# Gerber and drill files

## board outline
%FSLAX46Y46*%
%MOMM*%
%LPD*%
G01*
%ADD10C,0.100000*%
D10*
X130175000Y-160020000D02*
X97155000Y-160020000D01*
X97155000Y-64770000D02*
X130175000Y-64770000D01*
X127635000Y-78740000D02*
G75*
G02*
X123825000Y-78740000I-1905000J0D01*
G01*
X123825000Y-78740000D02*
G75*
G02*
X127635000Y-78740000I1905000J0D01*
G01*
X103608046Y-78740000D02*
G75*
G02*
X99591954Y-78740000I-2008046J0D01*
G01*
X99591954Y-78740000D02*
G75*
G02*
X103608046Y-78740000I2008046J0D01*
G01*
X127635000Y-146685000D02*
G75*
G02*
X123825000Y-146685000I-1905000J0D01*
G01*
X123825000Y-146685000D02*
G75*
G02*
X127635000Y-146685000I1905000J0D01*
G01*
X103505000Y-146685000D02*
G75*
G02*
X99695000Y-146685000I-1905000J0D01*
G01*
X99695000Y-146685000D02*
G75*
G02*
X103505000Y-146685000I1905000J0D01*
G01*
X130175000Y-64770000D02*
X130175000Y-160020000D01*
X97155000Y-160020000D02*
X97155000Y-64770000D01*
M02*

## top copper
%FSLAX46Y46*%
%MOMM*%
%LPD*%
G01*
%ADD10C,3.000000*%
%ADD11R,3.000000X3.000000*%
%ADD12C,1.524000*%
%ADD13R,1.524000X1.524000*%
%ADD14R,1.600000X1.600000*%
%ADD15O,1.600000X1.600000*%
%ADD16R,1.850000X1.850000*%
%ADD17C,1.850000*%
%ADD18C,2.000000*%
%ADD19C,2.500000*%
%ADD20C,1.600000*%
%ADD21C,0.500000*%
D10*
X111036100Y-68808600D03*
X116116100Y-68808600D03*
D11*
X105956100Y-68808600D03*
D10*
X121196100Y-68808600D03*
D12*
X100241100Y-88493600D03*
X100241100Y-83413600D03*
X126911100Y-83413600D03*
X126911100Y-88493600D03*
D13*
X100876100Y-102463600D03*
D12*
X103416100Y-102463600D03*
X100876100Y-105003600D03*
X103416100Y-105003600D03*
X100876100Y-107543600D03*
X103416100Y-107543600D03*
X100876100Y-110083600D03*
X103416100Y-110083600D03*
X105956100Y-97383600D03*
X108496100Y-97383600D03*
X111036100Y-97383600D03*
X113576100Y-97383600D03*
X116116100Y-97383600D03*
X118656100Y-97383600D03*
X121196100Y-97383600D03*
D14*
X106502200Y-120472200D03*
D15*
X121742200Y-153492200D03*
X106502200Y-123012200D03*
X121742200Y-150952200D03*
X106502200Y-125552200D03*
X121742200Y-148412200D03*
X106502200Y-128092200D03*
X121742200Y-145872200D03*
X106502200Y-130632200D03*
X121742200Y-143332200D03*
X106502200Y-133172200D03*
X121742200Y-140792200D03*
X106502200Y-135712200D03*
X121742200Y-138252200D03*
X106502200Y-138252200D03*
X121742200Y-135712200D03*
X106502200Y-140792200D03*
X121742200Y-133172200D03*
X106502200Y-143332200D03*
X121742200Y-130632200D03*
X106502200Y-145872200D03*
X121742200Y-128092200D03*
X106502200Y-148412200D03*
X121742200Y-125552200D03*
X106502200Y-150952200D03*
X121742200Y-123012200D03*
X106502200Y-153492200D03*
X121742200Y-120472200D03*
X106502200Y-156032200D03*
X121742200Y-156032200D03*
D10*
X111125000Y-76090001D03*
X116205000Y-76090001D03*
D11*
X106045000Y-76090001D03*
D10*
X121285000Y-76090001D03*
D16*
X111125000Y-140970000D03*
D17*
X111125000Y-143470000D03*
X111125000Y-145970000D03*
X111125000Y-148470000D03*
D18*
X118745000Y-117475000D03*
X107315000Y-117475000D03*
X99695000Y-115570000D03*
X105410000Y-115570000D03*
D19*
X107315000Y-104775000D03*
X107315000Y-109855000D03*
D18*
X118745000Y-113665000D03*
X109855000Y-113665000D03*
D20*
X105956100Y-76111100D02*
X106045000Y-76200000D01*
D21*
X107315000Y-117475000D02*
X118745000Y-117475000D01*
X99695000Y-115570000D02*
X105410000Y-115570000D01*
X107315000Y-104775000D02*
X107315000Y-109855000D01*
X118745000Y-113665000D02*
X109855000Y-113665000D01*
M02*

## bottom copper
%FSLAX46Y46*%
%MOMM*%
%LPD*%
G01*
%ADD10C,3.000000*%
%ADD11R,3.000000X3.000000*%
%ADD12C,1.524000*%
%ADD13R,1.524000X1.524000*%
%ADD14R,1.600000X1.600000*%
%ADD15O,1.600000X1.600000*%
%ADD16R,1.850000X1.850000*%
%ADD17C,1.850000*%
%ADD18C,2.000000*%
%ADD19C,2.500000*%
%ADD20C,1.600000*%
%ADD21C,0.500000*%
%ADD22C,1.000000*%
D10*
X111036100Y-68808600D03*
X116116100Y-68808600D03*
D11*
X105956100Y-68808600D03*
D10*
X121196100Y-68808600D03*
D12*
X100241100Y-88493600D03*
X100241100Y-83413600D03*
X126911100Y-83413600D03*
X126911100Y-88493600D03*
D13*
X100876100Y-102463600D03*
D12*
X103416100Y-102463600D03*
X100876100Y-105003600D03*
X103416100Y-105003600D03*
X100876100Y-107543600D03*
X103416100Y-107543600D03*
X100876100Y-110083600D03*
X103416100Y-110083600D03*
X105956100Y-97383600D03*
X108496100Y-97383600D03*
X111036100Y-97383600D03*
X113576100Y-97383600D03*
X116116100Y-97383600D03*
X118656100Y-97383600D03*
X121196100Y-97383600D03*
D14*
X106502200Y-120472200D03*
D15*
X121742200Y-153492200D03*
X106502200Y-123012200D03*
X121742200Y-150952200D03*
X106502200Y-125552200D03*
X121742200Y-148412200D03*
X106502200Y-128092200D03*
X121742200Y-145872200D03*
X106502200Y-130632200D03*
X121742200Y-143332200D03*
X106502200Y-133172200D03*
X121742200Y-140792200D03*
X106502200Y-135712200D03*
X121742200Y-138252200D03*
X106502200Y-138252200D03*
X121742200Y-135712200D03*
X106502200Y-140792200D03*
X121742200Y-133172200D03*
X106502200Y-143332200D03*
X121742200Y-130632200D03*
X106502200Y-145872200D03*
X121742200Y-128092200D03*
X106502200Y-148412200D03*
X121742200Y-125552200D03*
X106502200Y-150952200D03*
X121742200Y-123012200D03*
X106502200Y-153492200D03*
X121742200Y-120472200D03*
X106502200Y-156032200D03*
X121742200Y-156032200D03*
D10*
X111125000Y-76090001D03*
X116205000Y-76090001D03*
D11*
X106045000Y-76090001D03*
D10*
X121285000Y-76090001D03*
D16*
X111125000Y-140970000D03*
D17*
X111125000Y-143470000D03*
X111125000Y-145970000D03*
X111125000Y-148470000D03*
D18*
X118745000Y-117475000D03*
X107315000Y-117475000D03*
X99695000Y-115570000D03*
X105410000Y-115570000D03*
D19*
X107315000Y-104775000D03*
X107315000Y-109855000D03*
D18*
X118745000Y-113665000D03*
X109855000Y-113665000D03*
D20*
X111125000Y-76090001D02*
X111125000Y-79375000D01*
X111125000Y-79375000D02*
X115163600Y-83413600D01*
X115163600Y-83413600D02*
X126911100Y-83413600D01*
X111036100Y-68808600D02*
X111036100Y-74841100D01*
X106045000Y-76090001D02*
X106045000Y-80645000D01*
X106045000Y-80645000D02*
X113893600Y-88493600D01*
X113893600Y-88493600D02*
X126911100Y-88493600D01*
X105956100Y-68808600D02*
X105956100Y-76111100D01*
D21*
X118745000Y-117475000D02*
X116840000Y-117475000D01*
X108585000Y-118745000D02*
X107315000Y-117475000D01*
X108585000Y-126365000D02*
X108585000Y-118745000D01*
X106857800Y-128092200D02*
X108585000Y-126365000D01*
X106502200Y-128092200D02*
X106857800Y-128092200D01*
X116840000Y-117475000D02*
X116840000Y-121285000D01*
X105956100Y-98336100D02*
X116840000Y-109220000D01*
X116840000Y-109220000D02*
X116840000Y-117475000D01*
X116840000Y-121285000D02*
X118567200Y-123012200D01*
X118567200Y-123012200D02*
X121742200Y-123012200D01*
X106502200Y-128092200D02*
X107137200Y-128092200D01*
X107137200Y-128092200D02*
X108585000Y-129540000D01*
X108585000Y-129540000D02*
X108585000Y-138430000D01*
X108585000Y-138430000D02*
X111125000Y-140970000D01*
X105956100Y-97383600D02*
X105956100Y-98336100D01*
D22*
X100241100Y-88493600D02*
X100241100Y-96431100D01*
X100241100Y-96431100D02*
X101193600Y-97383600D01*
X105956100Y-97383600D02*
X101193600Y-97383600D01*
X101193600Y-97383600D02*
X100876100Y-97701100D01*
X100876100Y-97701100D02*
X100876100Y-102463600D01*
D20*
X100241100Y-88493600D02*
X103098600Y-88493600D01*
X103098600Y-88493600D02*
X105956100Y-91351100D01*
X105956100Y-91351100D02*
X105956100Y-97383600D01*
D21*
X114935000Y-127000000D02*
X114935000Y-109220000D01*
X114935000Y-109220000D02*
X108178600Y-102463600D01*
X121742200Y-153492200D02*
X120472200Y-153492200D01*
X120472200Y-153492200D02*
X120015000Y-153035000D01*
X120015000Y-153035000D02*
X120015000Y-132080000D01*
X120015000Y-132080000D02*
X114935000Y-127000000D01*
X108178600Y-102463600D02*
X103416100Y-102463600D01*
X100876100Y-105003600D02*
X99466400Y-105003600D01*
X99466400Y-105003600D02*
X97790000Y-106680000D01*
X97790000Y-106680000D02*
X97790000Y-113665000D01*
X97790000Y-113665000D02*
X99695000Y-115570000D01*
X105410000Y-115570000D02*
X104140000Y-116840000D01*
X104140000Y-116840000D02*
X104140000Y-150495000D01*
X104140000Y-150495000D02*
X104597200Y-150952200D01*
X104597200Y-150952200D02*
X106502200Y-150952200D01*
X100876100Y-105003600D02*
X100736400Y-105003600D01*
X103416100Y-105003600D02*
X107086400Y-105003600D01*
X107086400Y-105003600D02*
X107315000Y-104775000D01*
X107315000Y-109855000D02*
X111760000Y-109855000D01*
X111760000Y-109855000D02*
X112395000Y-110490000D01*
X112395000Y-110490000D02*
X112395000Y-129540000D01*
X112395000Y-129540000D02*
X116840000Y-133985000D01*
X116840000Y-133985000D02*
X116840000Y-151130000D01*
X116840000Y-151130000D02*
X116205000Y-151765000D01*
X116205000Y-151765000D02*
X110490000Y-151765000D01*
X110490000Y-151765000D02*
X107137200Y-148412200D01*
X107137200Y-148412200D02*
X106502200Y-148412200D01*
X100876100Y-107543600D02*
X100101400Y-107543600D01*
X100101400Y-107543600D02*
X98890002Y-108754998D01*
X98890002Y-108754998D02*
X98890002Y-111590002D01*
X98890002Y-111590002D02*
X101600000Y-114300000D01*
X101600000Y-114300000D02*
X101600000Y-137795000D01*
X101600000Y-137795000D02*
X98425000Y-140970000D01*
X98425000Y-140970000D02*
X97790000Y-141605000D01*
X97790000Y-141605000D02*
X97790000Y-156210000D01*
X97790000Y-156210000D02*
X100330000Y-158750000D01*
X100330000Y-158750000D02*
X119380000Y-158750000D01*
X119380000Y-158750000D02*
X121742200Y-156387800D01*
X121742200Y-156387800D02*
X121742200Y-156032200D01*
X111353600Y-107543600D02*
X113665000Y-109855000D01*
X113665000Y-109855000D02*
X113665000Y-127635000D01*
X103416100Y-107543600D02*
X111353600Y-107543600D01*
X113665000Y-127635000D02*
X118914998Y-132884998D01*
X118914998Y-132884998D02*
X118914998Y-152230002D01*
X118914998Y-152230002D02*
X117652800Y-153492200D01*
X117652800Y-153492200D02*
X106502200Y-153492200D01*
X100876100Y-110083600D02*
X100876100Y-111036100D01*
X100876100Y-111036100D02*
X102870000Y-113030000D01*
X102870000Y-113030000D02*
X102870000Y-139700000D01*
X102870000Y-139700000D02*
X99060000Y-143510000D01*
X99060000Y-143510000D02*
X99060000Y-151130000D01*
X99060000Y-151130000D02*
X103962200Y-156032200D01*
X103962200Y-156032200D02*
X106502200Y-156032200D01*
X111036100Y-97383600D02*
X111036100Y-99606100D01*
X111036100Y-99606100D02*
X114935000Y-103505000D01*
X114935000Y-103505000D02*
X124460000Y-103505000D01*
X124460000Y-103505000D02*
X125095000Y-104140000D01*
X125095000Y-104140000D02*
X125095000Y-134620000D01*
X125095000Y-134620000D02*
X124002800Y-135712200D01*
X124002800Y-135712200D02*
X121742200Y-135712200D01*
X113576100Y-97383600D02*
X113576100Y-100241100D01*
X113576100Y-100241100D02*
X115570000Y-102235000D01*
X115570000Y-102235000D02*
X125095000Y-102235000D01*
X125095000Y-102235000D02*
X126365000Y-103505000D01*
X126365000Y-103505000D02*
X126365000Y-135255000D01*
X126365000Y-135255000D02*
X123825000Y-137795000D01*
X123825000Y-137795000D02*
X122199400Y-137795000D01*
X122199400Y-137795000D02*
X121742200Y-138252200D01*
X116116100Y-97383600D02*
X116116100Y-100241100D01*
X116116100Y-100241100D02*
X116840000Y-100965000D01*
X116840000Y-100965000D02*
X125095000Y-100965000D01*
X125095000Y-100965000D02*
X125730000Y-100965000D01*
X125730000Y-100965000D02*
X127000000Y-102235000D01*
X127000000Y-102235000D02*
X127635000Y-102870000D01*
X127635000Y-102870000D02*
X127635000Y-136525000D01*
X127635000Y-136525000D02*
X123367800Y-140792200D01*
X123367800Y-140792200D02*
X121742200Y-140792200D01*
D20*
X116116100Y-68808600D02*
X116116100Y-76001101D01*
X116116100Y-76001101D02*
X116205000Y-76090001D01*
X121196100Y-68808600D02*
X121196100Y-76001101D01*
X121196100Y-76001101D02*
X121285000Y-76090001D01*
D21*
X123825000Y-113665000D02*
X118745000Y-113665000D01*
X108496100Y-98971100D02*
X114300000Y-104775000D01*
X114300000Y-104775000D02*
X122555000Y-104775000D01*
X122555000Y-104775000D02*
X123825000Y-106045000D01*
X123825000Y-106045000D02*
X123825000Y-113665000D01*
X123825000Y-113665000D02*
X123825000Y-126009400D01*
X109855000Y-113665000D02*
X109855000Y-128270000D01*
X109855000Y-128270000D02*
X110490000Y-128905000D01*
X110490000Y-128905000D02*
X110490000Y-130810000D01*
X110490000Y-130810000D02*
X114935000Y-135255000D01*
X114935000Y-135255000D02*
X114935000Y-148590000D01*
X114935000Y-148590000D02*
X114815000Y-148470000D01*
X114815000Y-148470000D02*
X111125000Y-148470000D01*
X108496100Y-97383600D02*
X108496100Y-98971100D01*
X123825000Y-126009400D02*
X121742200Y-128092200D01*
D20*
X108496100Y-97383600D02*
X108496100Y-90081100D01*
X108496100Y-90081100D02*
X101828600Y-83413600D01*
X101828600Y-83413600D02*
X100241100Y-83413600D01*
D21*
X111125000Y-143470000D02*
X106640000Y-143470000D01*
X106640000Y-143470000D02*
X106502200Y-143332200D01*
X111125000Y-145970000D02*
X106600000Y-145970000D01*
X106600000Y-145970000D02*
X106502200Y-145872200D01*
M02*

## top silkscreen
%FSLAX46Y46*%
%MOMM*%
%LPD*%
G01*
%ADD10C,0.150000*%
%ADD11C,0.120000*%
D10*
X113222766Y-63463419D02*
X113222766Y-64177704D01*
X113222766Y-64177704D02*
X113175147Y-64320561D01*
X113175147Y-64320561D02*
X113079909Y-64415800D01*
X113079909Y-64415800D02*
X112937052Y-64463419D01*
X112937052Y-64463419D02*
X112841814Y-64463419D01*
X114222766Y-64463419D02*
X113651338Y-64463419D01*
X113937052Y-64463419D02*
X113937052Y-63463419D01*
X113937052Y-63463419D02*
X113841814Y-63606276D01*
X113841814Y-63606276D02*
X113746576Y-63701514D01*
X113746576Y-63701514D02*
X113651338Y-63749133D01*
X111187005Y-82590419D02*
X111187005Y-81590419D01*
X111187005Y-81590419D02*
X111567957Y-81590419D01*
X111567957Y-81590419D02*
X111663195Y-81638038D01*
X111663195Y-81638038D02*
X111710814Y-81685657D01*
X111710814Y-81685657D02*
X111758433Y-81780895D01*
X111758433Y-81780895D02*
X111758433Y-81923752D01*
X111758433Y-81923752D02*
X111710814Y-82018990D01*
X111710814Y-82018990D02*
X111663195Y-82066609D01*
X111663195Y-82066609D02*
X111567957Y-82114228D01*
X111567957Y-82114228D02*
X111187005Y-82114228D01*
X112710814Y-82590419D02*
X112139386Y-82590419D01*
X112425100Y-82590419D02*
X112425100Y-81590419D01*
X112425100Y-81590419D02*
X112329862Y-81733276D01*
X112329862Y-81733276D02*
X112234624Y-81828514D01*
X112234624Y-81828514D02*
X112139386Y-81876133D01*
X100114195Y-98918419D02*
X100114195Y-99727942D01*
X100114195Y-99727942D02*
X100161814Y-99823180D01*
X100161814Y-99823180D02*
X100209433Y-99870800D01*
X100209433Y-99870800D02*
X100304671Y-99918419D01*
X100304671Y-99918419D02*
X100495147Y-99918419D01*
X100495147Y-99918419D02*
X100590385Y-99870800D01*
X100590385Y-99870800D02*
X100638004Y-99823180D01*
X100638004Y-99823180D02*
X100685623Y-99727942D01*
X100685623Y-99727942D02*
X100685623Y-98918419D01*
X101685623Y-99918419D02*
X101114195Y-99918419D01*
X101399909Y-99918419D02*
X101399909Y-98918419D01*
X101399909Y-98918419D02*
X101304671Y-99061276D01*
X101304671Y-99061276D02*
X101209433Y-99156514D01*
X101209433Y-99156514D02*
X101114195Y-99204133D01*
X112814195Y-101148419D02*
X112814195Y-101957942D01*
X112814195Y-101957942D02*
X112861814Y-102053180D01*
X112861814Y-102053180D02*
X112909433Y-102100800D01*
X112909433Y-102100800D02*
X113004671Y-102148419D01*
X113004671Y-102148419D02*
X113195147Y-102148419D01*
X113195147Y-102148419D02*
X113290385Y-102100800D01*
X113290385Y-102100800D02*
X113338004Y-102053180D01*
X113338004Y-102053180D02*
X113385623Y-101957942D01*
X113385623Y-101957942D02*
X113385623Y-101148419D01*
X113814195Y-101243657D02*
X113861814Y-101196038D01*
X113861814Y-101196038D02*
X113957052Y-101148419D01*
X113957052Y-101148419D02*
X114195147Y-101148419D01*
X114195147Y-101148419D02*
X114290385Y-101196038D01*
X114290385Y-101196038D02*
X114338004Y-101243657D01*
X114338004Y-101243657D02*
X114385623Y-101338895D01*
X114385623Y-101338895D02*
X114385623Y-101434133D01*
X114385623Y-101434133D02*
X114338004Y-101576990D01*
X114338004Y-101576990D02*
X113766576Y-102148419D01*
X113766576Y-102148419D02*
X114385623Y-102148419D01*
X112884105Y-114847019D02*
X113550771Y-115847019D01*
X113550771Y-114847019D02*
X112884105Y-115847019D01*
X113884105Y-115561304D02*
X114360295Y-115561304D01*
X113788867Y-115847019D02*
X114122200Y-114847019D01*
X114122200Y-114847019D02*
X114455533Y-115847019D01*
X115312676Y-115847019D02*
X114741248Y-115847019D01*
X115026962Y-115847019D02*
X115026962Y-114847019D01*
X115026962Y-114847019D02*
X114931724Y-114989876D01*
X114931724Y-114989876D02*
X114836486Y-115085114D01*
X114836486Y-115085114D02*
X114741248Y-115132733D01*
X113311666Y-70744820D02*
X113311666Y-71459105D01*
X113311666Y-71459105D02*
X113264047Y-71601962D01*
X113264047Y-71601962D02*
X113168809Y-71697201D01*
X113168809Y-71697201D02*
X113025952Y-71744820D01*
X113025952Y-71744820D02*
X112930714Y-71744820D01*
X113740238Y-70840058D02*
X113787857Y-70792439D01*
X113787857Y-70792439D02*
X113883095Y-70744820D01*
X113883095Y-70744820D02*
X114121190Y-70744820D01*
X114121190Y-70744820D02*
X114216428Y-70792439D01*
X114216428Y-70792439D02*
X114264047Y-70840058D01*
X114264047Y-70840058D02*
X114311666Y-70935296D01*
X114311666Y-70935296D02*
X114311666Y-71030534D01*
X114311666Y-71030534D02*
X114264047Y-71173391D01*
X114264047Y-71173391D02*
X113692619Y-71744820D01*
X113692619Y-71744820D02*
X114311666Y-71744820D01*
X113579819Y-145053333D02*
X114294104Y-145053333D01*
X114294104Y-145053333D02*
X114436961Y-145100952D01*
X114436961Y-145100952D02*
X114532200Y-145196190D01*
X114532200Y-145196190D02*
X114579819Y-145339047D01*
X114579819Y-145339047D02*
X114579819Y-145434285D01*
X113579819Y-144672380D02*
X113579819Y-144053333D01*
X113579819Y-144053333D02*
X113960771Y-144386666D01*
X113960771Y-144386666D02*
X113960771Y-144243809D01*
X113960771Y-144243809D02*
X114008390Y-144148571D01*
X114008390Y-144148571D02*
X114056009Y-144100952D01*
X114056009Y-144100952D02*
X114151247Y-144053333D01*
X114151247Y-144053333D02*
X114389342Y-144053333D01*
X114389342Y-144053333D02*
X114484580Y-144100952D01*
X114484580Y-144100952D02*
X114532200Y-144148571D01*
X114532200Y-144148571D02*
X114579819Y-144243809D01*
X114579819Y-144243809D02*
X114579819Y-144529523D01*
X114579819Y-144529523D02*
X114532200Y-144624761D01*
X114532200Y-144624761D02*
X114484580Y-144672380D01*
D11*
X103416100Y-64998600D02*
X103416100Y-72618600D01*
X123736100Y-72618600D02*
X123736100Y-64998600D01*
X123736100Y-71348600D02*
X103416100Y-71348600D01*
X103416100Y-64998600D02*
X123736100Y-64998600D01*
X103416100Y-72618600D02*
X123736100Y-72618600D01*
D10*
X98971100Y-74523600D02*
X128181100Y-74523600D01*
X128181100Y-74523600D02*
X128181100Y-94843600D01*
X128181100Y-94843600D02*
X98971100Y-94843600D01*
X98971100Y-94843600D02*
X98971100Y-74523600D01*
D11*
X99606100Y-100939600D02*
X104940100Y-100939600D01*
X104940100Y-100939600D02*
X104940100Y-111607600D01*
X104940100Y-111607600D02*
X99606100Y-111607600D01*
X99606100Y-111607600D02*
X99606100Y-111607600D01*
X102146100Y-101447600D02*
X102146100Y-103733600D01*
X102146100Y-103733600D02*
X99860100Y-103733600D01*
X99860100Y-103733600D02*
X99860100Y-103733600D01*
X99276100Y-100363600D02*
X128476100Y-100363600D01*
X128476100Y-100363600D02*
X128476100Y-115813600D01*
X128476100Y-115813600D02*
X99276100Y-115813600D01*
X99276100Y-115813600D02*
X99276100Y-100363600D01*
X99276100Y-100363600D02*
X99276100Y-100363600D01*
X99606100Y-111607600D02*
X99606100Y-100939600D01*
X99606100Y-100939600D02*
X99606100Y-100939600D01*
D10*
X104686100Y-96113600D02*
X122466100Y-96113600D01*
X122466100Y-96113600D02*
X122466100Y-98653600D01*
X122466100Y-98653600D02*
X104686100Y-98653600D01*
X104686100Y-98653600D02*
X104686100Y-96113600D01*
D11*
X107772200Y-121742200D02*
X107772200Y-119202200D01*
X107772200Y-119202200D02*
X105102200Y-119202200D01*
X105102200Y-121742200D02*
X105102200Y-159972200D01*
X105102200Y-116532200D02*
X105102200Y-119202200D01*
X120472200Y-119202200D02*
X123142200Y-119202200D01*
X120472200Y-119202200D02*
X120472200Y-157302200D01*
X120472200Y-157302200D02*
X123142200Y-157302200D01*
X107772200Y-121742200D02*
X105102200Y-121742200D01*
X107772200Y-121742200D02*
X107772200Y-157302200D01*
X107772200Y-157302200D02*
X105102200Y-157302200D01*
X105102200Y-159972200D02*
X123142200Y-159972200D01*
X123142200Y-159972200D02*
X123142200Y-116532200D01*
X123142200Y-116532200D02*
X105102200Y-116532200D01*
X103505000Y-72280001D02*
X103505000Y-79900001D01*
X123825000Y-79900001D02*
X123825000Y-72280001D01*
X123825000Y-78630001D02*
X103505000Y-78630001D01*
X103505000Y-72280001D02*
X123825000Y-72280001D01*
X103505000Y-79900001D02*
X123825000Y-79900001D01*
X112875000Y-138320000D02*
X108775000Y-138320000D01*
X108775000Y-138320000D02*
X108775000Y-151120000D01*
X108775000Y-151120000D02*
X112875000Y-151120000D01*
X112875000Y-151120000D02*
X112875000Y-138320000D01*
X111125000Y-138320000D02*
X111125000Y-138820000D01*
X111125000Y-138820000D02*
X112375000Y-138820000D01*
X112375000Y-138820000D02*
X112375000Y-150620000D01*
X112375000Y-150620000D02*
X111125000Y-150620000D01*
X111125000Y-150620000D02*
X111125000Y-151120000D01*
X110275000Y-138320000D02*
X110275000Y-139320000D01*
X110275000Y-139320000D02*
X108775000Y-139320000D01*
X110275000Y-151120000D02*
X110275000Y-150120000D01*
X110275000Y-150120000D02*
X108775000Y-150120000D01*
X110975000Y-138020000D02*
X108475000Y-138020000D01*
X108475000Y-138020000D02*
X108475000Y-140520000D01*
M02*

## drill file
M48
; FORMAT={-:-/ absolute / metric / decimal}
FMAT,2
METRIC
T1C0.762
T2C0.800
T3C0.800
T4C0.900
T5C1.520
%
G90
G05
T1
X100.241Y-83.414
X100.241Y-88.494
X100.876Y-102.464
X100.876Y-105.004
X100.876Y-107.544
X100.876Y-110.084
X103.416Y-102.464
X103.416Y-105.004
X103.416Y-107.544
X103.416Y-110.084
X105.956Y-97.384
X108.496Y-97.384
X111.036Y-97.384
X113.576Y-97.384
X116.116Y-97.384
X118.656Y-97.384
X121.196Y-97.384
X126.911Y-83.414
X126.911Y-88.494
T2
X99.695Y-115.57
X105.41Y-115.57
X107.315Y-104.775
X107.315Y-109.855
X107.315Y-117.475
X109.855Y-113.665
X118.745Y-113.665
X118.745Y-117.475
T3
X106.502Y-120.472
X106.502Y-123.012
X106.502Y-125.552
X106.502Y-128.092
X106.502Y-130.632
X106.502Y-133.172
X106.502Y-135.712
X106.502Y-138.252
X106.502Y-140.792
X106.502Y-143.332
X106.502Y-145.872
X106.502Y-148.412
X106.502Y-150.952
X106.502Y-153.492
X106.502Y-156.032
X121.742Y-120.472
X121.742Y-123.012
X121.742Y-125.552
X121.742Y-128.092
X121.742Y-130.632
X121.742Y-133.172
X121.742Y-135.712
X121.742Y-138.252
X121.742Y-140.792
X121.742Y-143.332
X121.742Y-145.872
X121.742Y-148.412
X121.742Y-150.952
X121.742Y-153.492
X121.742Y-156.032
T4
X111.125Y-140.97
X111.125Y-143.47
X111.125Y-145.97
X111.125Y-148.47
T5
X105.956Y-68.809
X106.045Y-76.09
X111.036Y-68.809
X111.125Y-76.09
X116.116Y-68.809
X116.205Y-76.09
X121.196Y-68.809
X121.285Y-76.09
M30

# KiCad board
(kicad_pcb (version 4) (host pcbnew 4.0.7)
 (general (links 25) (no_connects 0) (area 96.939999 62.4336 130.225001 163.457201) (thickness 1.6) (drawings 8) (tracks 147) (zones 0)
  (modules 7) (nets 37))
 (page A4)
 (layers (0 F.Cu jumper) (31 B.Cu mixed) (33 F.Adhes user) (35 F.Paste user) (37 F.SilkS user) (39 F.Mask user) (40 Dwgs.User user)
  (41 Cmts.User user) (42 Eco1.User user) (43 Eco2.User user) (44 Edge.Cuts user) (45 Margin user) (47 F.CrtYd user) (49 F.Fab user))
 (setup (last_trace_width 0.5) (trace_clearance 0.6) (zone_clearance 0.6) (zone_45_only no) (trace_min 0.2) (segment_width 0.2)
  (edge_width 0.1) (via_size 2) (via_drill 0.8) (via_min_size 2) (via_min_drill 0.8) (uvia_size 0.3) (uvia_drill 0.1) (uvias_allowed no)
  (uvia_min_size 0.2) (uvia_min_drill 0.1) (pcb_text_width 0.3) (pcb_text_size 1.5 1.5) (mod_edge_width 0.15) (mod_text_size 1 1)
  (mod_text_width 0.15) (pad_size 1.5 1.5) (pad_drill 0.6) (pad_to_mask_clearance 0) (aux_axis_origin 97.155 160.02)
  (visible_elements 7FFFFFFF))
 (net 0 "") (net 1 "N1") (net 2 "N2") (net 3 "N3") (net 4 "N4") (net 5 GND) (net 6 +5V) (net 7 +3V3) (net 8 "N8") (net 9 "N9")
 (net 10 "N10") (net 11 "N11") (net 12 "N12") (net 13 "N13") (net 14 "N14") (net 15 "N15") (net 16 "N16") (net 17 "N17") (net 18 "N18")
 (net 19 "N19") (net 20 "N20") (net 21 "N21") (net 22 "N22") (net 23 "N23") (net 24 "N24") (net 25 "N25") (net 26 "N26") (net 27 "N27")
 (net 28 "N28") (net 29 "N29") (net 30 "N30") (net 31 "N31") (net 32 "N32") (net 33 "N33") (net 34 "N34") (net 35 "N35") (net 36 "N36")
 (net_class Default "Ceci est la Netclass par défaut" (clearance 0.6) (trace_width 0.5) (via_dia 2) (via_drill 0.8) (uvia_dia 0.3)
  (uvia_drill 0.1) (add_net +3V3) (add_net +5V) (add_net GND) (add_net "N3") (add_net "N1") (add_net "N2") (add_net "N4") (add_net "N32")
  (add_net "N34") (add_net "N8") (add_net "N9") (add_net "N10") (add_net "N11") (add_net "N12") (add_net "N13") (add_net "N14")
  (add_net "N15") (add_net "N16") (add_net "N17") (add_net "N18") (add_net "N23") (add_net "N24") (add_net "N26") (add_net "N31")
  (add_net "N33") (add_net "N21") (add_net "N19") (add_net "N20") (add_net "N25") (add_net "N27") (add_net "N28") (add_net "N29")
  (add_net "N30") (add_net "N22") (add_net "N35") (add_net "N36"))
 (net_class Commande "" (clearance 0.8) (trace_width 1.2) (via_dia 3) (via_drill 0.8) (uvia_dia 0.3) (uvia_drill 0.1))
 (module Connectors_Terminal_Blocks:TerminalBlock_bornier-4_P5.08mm (layer F.Cu) (at 105.9561 68.8086)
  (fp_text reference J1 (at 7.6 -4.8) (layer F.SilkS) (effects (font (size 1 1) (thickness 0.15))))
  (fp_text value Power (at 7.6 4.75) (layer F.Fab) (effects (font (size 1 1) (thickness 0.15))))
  (fp_line (start -2.54 -3.81) (end -2.54 3.81) (layer F.SilkS) (width 0.12))
  (fp_line (start 17.78 3.81) (end 17.78 -3.81) (layer F.SilkS) (width 0.12))
  (fp_line (start 17.78 2.54) (end -2.54 2.54) (layer F.SilkS) (width 0.12))
  (fp_line (start -2.54 -3.81) (end 17.78 -3.81) (layer F.SilkS) (width 0.12))
  (fp_line (start -2.54 3.81) (end 17.78 3.81) (layer F.SilkS) (width 0.12))
  (pad 2 thru_hole circle (at 5.08 0) (size 3 3) (drill 1.52) (layers *.Cu *.Mask) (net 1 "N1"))
  (pad 3 thru_hole circle (at 10.16 0) (size 3 3) (drill 1.52) (layers *.Cu *.Mask) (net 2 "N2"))
  (pad 1 thru_hole rect (at 0 0) (size 3 3) (drill 1.52) (layers *.Cu *.Mask) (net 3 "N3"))
  (pad 4 thru_hole circle (at 15.24 0) (size 3 3) (drill 1.52) (layers *.Cu *.Mask) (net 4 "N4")))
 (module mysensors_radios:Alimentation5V (layer F.Cu) (at 112.9411 84.6836)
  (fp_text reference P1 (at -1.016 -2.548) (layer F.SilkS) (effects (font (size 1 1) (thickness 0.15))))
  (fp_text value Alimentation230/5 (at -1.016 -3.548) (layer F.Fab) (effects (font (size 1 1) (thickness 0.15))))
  (fp_line (start -13.97 -10.16) (end 15.24 -10.16) (layer F.SilkS) (width 0.15))
  (fp_line (start 15.24 -10.16) (end 15.24 10.16) (layer F.SilkS) (width 0.15))
  (fp_line (start 15.24 10.16) (end -13.97 10.16) (layer F.SilkS) (width 0.15))
  (fp_line (start -13.97 10.16) (end -13.97 -10.16) (layer F.SilkS) (width 0.15))
  (pad 4 thru_hole circle (at -12.7 3.81) (size 1.524 1.524) (drill 0.762) (layers *.Cu *.Mask) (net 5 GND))
  (pad 3 thru_hole circle (at -12.7 -1.27) (size 1.524 1.524) (drill 0.762) (layers *.Cu *.Mask) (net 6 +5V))
  (pad 1 thru_hole circle (at 13.97 -1.27) (size 1.524 1.524) (drill 0.762) (layers *.Cu *.Mask) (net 1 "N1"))
  (pad 2 thru_hole circle (at 13.97 3.81) (size 1.524 1.524) (drill 0.762) (layers *.Cu *.Mask) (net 3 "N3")))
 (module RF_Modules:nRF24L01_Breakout (layer F.Cu) (at 100.8761 102.4636)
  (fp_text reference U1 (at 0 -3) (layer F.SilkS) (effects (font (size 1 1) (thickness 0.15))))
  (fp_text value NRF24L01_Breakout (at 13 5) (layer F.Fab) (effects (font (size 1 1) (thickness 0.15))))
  (fp_line (start -1.27 -1.524) (end 4.064 -1.524) (layer F.SilkS) (width 0.12))
  (fp_line (start 4.064 -1.524) (end 4.064 9.144) (layer F.SilkS) (width 0.12))
  (fp_line (start 4.064 9.144) (end -1.27 9.144) (layer F.SilkS) (width 0.12))
  (fp_line (start -1.27 9.144) (end -1.27 9.144) (layer F.SilkS) (width 0.12))
  (fp_line (start 1.27 -1.016) (end 1.27 1.27) (layer F.SilkS) (width 0.12))
  (fp_line (start 1.27 1.27) (end -1.016 1.27) (layer F.SilkS) (width 0.12))
  (fp_line (start -1.016 1.27) (end -1.016 1.27) (layer F.SilkS) (width 0.12))
  (fp_line (start -1.6 -2.1) (end 27.6 -2.1) (layer F.SilkS) (width 0.12))
  (fp_line (start 27.6 -2.1) (end 27.6 13.35) (layer F.SilkS) (width 0.12))
  (fp_line (start 27.6 13.35) (end -1.6 13.35) (layer F.SilkS) (width 0.12))
  (fp_line (start -1.6 13.35) (end -1.6 -2.1) (layer F.SilkS) (width 0.12))
  (fp_line (start -1.6 -2.1) (end -1.6 -2.1) (layer F.SilkS) (width 0.12))
  (fp_line (start -1.27 9.144) (end -1.27 -1.524) (layer F.SilkS) (width 0.12))
  (fp_line (start -1.27 -1.524) (end -1.27 -1.524) (layer F.SilkS) (width 0.12))
  (pad 1 thru_hole rect (at 0 0) (size 1.524 1.524) (drill 0.762) (layers *.Cu *.Mask) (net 5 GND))
  (pad 2 thru_hole circle (at 2.54 0) (size 1.524 1.524) (drill 0.762) (layers *.Cu *.Mask) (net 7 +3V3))
  (pad 3 thru_hole circle (at 0 2.54) (size 1.524 1.524) (drill 0.762) (layers *.Cu *.Mask) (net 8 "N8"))
  (pad 4 thru_hole circle (at 2.54 2.54) (size 1.524 1.524) (drill 0.762) (layers *.Cu *.Mask) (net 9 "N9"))
  (pad 5 thru_hole circle (at 0 5.08) (size 1.524 1.524) (drill 0.762) (layers *.Cu *.Mask) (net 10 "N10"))
  (pad 6 thru_hole circle (at 2.54 5.08) (size 1.524 1.524) (drill 0.762) (layers *.Cu *.Mask) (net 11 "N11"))
  (pad 7 thru_hole circle (at 0 7.62) (size 1.524 1.524) (drill 0.762) (layers *.Cu *.Mask) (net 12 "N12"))
  (pad 8 thru_hole circle (at 2.54 7.62) (size 1.524 1.524) (drill 0.762) (layers *.Cu *.Mask) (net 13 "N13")))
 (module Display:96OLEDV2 (layer F.Cu) (at 105.9561 97.3836)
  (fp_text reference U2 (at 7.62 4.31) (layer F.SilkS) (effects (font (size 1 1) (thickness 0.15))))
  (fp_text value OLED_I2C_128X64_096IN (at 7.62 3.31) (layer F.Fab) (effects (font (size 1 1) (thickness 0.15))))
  (fp_line (start -1.27 -1.27) (end 16.51 -1.27) (layer F.SilkS) (width 0.15))
  (fp_line (start 16.51 -1.27) (end 16.51 1.27) (layer F.SilkS) (width 0.15))
  (fp_line (start 16.51 1.27) (end -1.27 1.27) (layer F.SilkS) (width 0.15))
  (fp_line (start -1.27 1.27) (end -1.27 -1.27) (layer F.SilkS) (width 0.15))
  (pad 1 thru_hole circle (at 0 0) (size 1.524 1.524) (drill 0.762) (layers *.Cu *.Mask) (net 5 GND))
  (pad 2 thru_hole circle (at 2.54 0) (size 1.524 1.524) (drill 0.762) (layers *.Cu *.Mask) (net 6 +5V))
  (pad 3 thru_hole circle (at 5.08 0) (size 1.524 1.524) (drill 0.762) (layers *.Cu *.Mask) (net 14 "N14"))
  (pad 4 thru_hole circle (at 7.62 0) (size 1.524 1.524) (drill 0.762) (layers *.Cu *.Mask) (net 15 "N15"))
  (pad 5 thru_hole circle (at 10.16 0) (size 1.524 1.524) (drill 0.762) (layers *.Cu *.Mask) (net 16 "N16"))
  (pad 6 thru_hole circle (at 12.7 0) (size 1.524 1.524) (drill 0.762) (layers *.Cu *.Mask) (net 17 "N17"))
  (pad 7 thru_hole circle (at 15.24 0) (size 1.524 1.524) (drill 0.762) (layers *.Cu *.Mask) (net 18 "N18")))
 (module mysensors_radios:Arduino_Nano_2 (layer F.Cu) (at 106.5022 120.4722)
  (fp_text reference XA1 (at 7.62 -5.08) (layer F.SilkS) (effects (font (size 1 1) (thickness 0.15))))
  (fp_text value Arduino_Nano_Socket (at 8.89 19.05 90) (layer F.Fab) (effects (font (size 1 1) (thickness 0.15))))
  (fp_line (start 1.27 1.27) (end 1.27 -1.27) (layer F.SilkS) (width 0.12))
  (fp_line (start 1.27 -1.27) (end -1.4 -1.27) (layer F.SilkS) (width 0.12))
  (fp_line (start -1.4 1.27) (end -1.4 39.5) (layer F.SilkS) (width 0.12))
  (fp_line (start -1.4 -3.94) (end -1.4 -1.27) (layer F.SilkS) (width 0.12))
  (fp_line (start 13.97 -1.27) (end 16.64 -1.27) (layer F.SilkS) (width 0.12))
  (fp_line (start 13.97 -1.27) (end 13.97 36.83) (layer F.SilkS) (width 0.12))
  (fp_line (start 13.97 36.83) (end 16.64 36.83) (layer F.SilkS) (width 0.12))
  (fp_line (start 1.27 1.27) (end -1.4 1.27) (layer F.SilkS) (width 0.12))
  (fp_line (start 1.27 1.27) (end 1.27 36.83) (layer F.SilkS) (width 0.12))
  (fp_line (start 1.27 36.83) (end -1.4 36.83) (layer F.SilkS) (width 0.12))
  (fp_line (start -1.4 39.5) (end 16.64 39.5) (layer F.SilkS) (width 0.12))
  (fp_line (start 16.64 39.5) (end 16.64 -3.94) (layer F.SilkS) (width 0.12))
  (fp_line (start 16.64 -3.94) (end -1.4 -3.94) (layer F.SilkS) (width 0.12))
  (pad D0 thru_hole rect (at 0 0) (size 1.6 1.6) (drill 0.8) (layers *.Cu *.Mask) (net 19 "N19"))
  (pad 3V3 thru_hole oval (at 15.24 33.02) (size 1.6 1.6) (drill 0.8) (layers *.Cu *.Mask) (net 7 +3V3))
  (pad D1 thru_hole oval (at 0 2.54) (size 1.6 1.6) (drill 0.8) (layers *.Cu *.Mask) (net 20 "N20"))
  (pad AREF thru_hole oval (at 15.24 30.48) (size 1.6 1.6) (drill 0.8) (layers *.Cu *.Mask) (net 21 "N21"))
  (pad RST1 thru_hole oval (at 0 5.08) (size 1.6 1.6) (drill 0.8) (layers *.Cu *.Mask) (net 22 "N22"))
  (pad A0 thru_hole oval (at 15.24 27.94) (size 1.6 1.6) (drill 0.8) (layers *.Cu *.Mask) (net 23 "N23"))
  (pad GND1 thru_hole oval (at 0 7.62) (size 1.6 1.6) (drill 0.8) (layers *.Cu *.Mask) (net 5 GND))
  (pad A1 thru_hole oval (at 15.24 25.4) (size 1.6 1.6) (drill 0.8) (layers *.Cu *.Mask) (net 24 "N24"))
  (pad D2 thru_hole oval (at 0 10.16) (size 1.6 1.6) (drill 0.8) (layers *.Cu *.Mask) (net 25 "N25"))
  (pad A2 thru_hole oval (at 15.24 22.86) (size 1.6 1.6) (drill 0.8) (layers *.Cu *.Mask) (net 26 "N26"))
  (pad D3 thru_hole oval (at 0 12.7) (size 1.6 1.6) (drill 0.8) (layers *.Cu *.Mask) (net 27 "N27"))
  (pad A3 thru_hole oval (at 15.24 20.32) (size 1.6 1.6) (drill 0.8) (layers *.Cu *.Mask) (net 16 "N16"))
  (pad D4 thru_hole oval (at 0 15.24) (size 1.6 1.6) (drill 0.8) (layers *.Cu *.Mask) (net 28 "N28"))
  (pad A4 thru_hole oval (at 15.24 17.78) (size 1.6 1.6) (drill 0.8) (layers *.Cu *.Mask) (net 15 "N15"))
  (pad D5 thru_hole oval (at 0 17.78) (size 1.6 1.6) (drill 0.8) (layers *.Cu *.Mask) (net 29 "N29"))
  (pad A5 thru_hole oval (at 15.24 15.24) (size 1.6 1.6) (drill 0.8) (layers *.Cu *.Mask) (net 14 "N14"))
  (pad D6 thru_hole oval (at 0 20.32) (size 1.6 1.6) (drill 0.8) (layers *.Cu *.Mask) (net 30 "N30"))
  (pad A6 thru_hole oval (at 15.24 12.7) (size 1.6 1.6) (drill 0.8) (layers *.Cu *.Mask) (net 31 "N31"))
  (pad D7 thru_hole oval (at 0 22.86) (size 1.6 1.6) (drill 0.8) (layers *.Cu *.Mask) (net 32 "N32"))
  (pad A7 thru_hole oval (at 15.24 10.16) (size 1.6 1.6) (drill 0.8) (layers *.Cu *.Mask) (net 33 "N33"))
  (pad D8 thru_hole oval (at 0 25.4) (size 1.6 1.6) (drill 0.8) (layers *.Cu *.Mask) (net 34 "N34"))
  (pad 5V thru_hole oval (at 15.24 7.62) (size 1.6 1.6) (drill 0.8) (layers *.Cu *.Mask) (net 6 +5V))
  (pad D9 thru_hole oval (at 0 27.94) (size 1.6 1.6) (drill 0.8) (layers *.Cu *.Mask) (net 9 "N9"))
  (pad RST2 thru_hole oval (at 15.24 5.08) (size 1.6 1.6) (drill 0.8) (layers *.Cu *.Mask) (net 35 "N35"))
  (pad D10 thru_hole oval (at 0 30.48) (size 1.6 1.6) (drill 0.8) (layers *.Cu *.Mask) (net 8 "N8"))
  (pad GND2 thru_hole oval (at 15.24 2.54) (size 1.6 1.6) (drill 0.8) (layers *.Cu *.Mask) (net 5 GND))
  (pad D11 thru_hole oval (at 0 33.02) (size 1.6 1.6) (drill 0.8) (layers *.Cu *.Mask) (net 11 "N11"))
  (pad VIN thru_hole oval (at 15.24 0) (size 1.6 1.6) (drill 0.8) (layers *.Cu *.Mask) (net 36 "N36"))
  (pad D12 thru_hole oval (at 0 35.56) (size 1.6 1.6) (drill 0.8) (layers *.Cu *.Mask) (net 12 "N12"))
  (pad D13 thru_hole oval (at 15.24 35.56) (size 1.6 1.6) (drill 0.8) (layers *.Cu *.Mask) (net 10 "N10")))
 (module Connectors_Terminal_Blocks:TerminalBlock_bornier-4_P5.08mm (layer F.Cu) (at 106.045 76.090001)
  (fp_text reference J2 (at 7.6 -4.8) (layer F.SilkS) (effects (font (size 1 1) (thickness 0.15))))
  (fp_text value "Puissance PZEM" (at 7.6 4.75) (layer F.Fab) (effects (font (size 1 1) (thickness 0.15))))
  (fp_line (start -2.54 -3.81) (end -2.54 3.81) (layer F.SilkS) (width 0.12))
  (fp_line (start 17.78 3.81) (end 17.78 -3.81) (layer F.SilkS) (width 0.12))
  (fp_line (start 17.78 2.54) (end -2.54 2.54) (layer F.SilkS) (width 0.12))
  (fp_line (start -2.54 -3.81) (end 17.78 -3.81) (layer F.SilkS) (width 0.12))
  (fp_line (start -2.54 3.81) (end 17.78 3.81) (layer F.SilkS) (width 0.12))
  (pad 2 thru_hole circle (at 5.08 0) (size 3 3) (drill 1.52) (layers *.Cu *.Mask) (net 1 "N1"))
  (pad 3 thru_hole circle (at 10.16 0) (size 3 3) (drill 1.52) (layers *.Cu *.Mask) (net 2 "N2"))
  (pad 1 thru_hole rect (at 0 0) (size 3 3) (drill 1.52) (layers *.Cu *.Mask) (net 3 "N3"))
  (pad 4 thru_hole circle (at 15.24 0) (size 3 3) (drill 1.52) (layers *.Cu *.Mask) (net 4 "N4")))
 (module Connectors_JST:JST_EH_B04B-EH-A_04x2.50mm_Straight (layer F.Cu) (at 111.125 140.97 270)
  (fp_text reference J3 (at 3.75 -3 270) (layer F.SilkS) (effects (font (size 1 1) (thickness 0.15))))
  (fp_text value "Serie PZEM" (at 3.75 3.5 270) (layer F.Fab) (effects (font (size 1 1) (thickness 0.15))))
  (fp_line (start -2.65 -1.75) (end -2.65 2.35) (layer F.SilkS) (width 0.12))
  (fp_line (start -2.65 2.35) (end 10.15 2.35) (layer F.SilkS) (width 0.12))
  (fp_line (start 10.15 2.35) (end 10.15 -1.75) (layer F.SilkS) (width 0.12))
  (fp_line (start 10.15 -1.75) (end -2.65 -1.75) (layer F.SilkS) (width 0.12))
  (fp_line (start -2.65 0) (end -2.15 0) (layer F.SilkS) (width 0.12))
  (fp_line (start -2.15 0) (end -2.15 -1.25) (layer F.SilkS) (width 0.12))
  (fp_line (start -2.15 -1.25) (end 9.65 -1.25) (layer F.SilkS) (width 0.12))
  (fp_line (start 9.65 -1.25) (end 9.65 0) (layer F.SilkS) (width 0.12))
  (fp_line (start 9.65 0) (end 10.15 0) (layer F.SilkS) (width 0.12))
  (fp_line (start -2.65 0.85) (end -1.65 0.85) (layer F.SilkS) (width 0.12))
  (fp_line (start -1.65 0.85) (end -1.65 2.35) (layer F.SilkS) (width 0.12))
  (fp_line (start 10.15 0.85) (end 9.15 0.85) (layer F.SilkS) (width 0.12))
  (fp_line (start 9.15 0.85) (end 9.15 2.35) (layer F.SilkS) (width 0.12))
  (fp_line (start -2.95 0.15) (end -2.95 2.65) (layer F.SilkS) (width 0.12))
  (fp_line (start -2.95 2.65) (end -0.45 2.65) (layer F.SilkS) (width 0.12))
  (pad 1 thru_hole rect (at 0 0 270) (size 1.85 1.85) (drill 0.9) (layers *.Cu *.Mask) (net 5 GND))
  (pad 2 thru_hole circle (at 2.5 0 270) (size 1.85 1.85) (drill 0.9) (layers *.Cu *.Mask) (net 32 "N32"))
  (pad 3 thru_hole circle (at 5 0 270) (size 1.85 1.85) (drill 0.9) (layers *.Cu *.Mask) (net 34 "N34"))
  (pad 4 thru_hole circle (at 7.5 0 270) (size 1.85 1.85) (drill 0.9) (layers *.Cu *.Mask) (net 6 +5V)))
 (gr_line (start 130.175 160.02) (end 97.155 160.02) (angle 90) (layer Edge.Cuts) (width 0.1))
 (gr_line (start 97.155 64.77) (end 130.175 64.77) (angle 90) (layer Edge.Cuts) (width 0.1))
 (gr_circle (center 125.73 78.74) (end 127.635 78.74) (layer Edge.Cuts) (width 0.1))
 (gr_circle (center 101.6 78.74) (end 99.695 78.105) (layer Edge.Cuts) (width 0.1))
 (gr_circle (center 125.73 146.685) (end 127.635 146.685) (layer Edge.Cuts) (width 0.1))
 (gr_circle (center 101.6 146.685) (end 99.695 146.685) (layer Edge.Cuts) (width 0.1))
 (gr_line (start 130.175 64.77) (end 130.175 160.02) (angle 90) (layer Edge.Cuts) (width 0.1))
 (gr_line (start 97.155 160.02) (end 97.155 64.77) (angle 90) (layer Edge.Cuts) (width 0.1))
 (segment (start 111.125 76.090001) (end 111.125 79.375) (width 1.6) (layer B.Cu) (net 1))
 (segment (start 111.125 79.375) (end 115.1636 83.4136) (width 1.6) (layer B.Cu) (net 1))
 (segment (start 115.1636 83.4136) (end 126.9111 83.4136) (width 1.6) (layer B.Cu) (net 1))
 (segment (start 111.0361 68.8086) (end 111.0361 74.8411) (width 1.6) (layer B.Cu) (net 1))
 (segment (start 106.045 76.090001) (end 106.045 80.645) (width 1.6) (layer B.Cu) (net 3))
 (segment (start 106.045 80.645) (end 113.8936 88.4936) (width 1.6) (layer B.Cu) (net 3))
 (segment (start 113.8936 88.4936) (end 126.9111 88.4936) (width 1.6) (layer B.Cu) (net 3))
 (segment (start 105.9561 76.1111) (end 106.045 76.2) (width 1.6) (layer F.Cu) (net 3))
 (segment (start 105.9561 68.8086) (end 105.9561 76.1111) (width 1.6) (layer B.Cu) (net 3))
 (segment (start 118.745 117.475) (end 116.84 117.475) (width 0.5) (layer B.Cu) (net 5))
 (via (at 118.745 117.475) (size 2) (drill 0.8) (layers F.Cu B.Cu) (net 5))
 (segment (start 107.315 117.475) (end 118.745 117.475) (width 0.5) (layer F.Cu) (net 5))
 (via (at 107.315 117.475) (size 2) (drill 0.8) (layers F.Cu B.Cu) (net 5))
 (segment (start 108.585 118.745) (end 107.315 117.475) (width 0.5) (layer B.Cu) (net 5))
 (segment (start 108.585 126.365) (end 108.585 118.745) (width 0.5) (layer B.Cu) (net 5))
 (segment (start 106.8578 128.0922) (end 108.585 126.365) (width 0.5) (layer B.Cu) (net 5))
 (segment (start 106.5022 128.0922) (end 106.8578 128.0922) (width 0.5) (layer B.Cu) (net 5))
 (segment (start 116.84 117.475) (end 116.84 121.285) (width 0.5) (layer B.Cu) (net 5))
 (segment (start 105.9561 98.3361) (end 116.84 109.22) (width 0.5) (layer B.Cu) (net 5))
 (segment (start 116.84 109.22) (end 116.84 117.475) (width 0.5) (layer B.Cu) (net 5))
 (segment (start 116.84 121.285) (end 118.5672 123.0122) (width 0.5) (layer B.Cu) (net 5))
 (segment (start 118.5672 123.0122) (end 121.7422 123.0122) (width 0.5) (layer B.Cu) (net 5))
 (segment (start 106.5022 128.0922) (end 107.1372 128.0922) (width 0.5) (layer B.Cu) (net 5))
 (segment (start 107.1372 128.0922) (end 108.585 129.54) (width 0.5) (layer B.Cu) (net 5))
 (segment (start 108.585 129.54) (end 108.585 138.43) (width 0.5) (layer B.Cu) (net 5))
 (segment (start 108.585 138.43) (end 111.125 140.97) (width 0.5) (layer B.Cu) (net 5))
 (segment (start 105.9561 97.3836) (end 105.9561 98.3361) (width 0.5) (layer B.Cu) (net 5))
 (segment (start 100.2411 88.4936) (end 100.2411 96.4311) (width 1) (layer B.Cu) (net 5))
 (segment (start 100.2411 96.4311) (end 101.1936 97.3836) (width 1) (layer B.Cu) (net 5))
 (segment (start 105.9561 97.3836) (end 101.1936 97.3836) (width 1) (layer B.Cu) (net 5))
 (segment (start 101.1936 97.3836) (end 100.8761 97.7011) (width 1) (layer B.Cu) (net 5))
 (segment (start 100.8761 97.7011) (end 100.8761 102.4636) (width 1) (layer B.Cu) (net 5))
 (segment (start 100.2411 88.4936) (end 103.0986 88.4936) (width 1.6) (layer B.Cu) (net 5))
 (segment (start 103.0986 88.4936) (end 105.9561 91.3511) (width 1.6) (layer B.Cu) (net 5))
 (segment (start 105.9561 91.3511) (end 105.9561 97.3836) (width 1.6) (layer B.Cu) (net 5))
 (segment (start 114.935 127) (end 114.935 109.22) (width 0.5) (layer B.Cu) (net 7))
 (segment (start 114.935 109.22) (end 108.1786 102.4636) (width 0.5) (layer B.Cu) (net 7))
 (segment (start 121.7422 153.4922) (end 120.4722 153.4922) (width 0.5) (layer B.Cu) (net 7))
 (segment (start 120.4722 153.4922) (end 120.015 153.035) (width 0.5) (layer B.Cu) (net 7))
 (segment (start 120.015 153.035) (end 120.015 132.08) (width 0.5) (layer B.Cu) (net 7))
 (segment (start 120.015 132.08) (end 114.935 127) (width 0.5) (layer B.Cu) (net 7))
 (segment (start 108.1786 102.4636) (end 103.4161 102.4636) (width 0.5) (layer B.Cu) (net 7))
 (segment (start 100.8761 105.0036) (end 99.4664 105.0036) (width 0.5) (layer B.Cu) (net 8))
 (segment (start 99.4664 105.0036) (end 97.79 106.68) (width 0.5) (layer B.Cu) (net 8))
 (segment (start 97.79 106.68) (end 97.79 113.665) (width 0.5) (layer B.Cu) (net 8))
 (segment (start 97.79 113.665) (end 99.695 115.57) (width 0.5) (layer B.Cu) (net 8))
 (via (at 99.695 115.57) (size 2) (drill 0.8) (layers F.Cu B.Cu) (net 8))
 (segment (start 99.695 115.57) (end 105.41 115.57) (width 0.5) (layer F.Cu) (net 8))
 (via (at 105.41 115.57) (size 2) (drill 0.8) (layers F.Cu B.Cu) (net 8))
 (segment (start 105.41 115.57) (end 104.14 116.84) (width 0.5) (layer B.Cu) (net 8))
 (segment (start 104.14 116.84) (end 104.14 150.495) (width 0.5) (layer B.Cu) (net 8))
 (segment (start 104.14 150.495) (end 104.5972 150.9522) (width 0.5) (layer B.Cu) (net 8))
 (segment (start 104.5972 150.9522) (end 106.5022 150.9522) (width 0.5) (layer B.Cu) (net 8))
 (segment (start 100.8761 105.0036) (end 100.7364 105.0036) (width 0.5) (layer B.Cu) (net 8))
 (segment (start 103.4161 105.0036) (end 107.0864 105.0036) (width 0.5) (layer B.Cu) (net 9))
 (segment (start 107.0864 105.0036) (end 107.315 104.775) (width 0.5) (layer B.Cu) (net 9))
 (via (at 107.315 104.775) (size 2.5) (drill 0.8) (layers F.Cu B.Cu) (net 9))
 (segment (start 107.315 104.775) (end 107.315 109.855) (width 0.5) (layer F.Cu) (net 9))
 (via (at 107.315 109.855) (size 2.5) (drill 0.8) (layers F.Cu B.Cu) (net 9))
 (segment (start 107.315 109.855) (end 111.76 109.855) (width 0.5) (layer B.Cu) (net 9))
 (segment (start 111.76 109.855) (end 112.395 110.49) (width 0.5) (layer B.Cu) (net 9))
 (segment (start 112.395 110.49) (end 112.395 129.54) (width 0.5) (layer B.Cu) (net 9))
 (segment (start 112.395 129.54) (end 116.84 133.985) (width 0.5) (layer B.Cu) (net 9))
 (segment (start 116.84 133.985) (end 116.84 151.13) (width 0.5) (layer B.Cu) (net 9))
 (segment (start 116.84 151.13) (end 116.205 151.765) (width 0.5) (layer B.Cu) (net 9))
 (segment (start 116.205 151.765) (end 110.49 151.765) (width 0.5) (layer B.Cu) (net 9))
 (segment (start 110.49 151.765) (end 107.1372 148.4122) (width 0.5) (layer B.Cu) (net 9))
 (segment (start 107.1372 148.4122) (end 106.5022 148.4122) (width 0.5) (layer B.Cu) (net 9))
 (segment (start 100.8761 107.5436) (end 100.1014 107.5436) (width 0.5) (layer B.Cu) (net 10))
 (segment (start 100.1014 107.5436) (end 98.890002 108.754998) (width 0.5) (layer B.Cu) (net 10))
 (segment (start 98.890002 108.754998) (end 98.890002 111.590002) (width 0.5) (layer B.Cu) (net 10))
 (segment (start 98.890002 111.590002) (end 101.6 114.3) (width 0.5) (layer B.Cu) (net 10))
 (segment (start 101.6 114.3) (end 101.6 137.795) (width 0.5) (layer B.Cu) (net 10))
 (segment (start 101.6 137.795) (end 98.425 140.97) (width 0.5) (layer B.Cu) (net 10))
 (segment (start 98.425 140.97) (end 97.79 141.605) (width 0.5) (layer B.Cu) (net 10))
 (segment (start 97.79 141.605) (end 97.79 156.21) (width 0.5) (layer B.Cu) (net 10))
 (segment (start 97.79 156.21) (end 100.33 158.75) (width 0.5) (layer B.Cu) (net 10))
 (segment (start 100.33 158.75) (end 119.38 158.75) (width 0.5) (layer B.Cu) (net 10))
 (segment (start 119.38 158.75) (end 121.7422 156.3878) (width 0.5) (layer B.Cu) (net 10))
 (segment (start 121.7422 156.3878) (end 121.7422 156.0322) (width 0.5) (layer B.Cu) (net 10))
 (segment (start 111.3536 107.5436) (end 113.665 109.855) (width 0.5) (layer B.Cu) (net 11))
 (segment (start 113.665 109.855) (end 113.665 127.635) (width 0.5) (layer B.Cu) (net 11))
 (segment (start 103.4161 107.5436) (end 111.3536 107.5436) (width 0.5) (layer B.Cu) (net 11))
 (segment (start 113.665 127.635) (end 118.914998 132.884998) (width 0.5) (layer B.Cu) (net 11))
 (segment (start 118.914998 132.884998) (end 118.914998 152.230002) (width 0.5) (layer B.Cu) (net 11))
 (segment (start 118.914998 152.230002) (end 117.6528 153.4922) (width 0.5) (layer B.Cu) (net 11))
 (segment (start 117.6528 153.4922) (end 106.5022 153.4922) (width 0.5) (layer B.Cu) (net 11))
 (segment (start 100.8761 110.0836) (end 100.8761 111.0361) (width 0.5) (layer B.Cu) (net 12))
 (segment (start 100.8761 111.0361) (end 102.87 113.03) (width 0.5) (layer B.Cu) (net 12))
 (segment (start 102.87 113.03) (end 102.87 139.7) (width 0.5) (layer B.Cu) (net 12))
 (segment (start 102.87 139.7) (end 99.06 143.51) (width 0.5) (layer B.Cu) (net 12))
 (segment (start 99.06 143.51) (end 99.06 151.13) (width 0.5) (layer B.Cu) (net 12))
 (segment (start 99.06 151.13) (end 103.9622 156.0322) (width 0.5) (layer B.Cu) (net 12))
 (segment (start 103.9622 156.0322) (end 106.5022 156.0322) (width 0.5) (layer B.Cu) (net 12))
 (segment (start 111.0361 97.3836) (end 111.0361 99.6061) (width 0.5) (layer B.Cu) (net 14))
 (segment (start 111.0361 99.6061) (end 114.935 103.505) (width 0.5) (layer B.Cu) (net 14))
 (segment (start 114.935 103.505) (end 124.46 103.505) (width 0.5) (layer B.Cu) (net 14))
 (segment (start 124.46 103.505) (end 125.095 104.14) (width 0.5) (layer B.Cu) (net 14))
 (segment (start 125.095 104.14) (end 125.095 134.62) (width 0.5) (layer B.Cu) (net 14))
 (segment (start 125.095 134.62) (end 124.0028 135.7122) (width 0.5) (layer B.Cu) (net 14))
 (segment (start 124.0028 135.7122) (end 121.7422 135.7122) (width 0.5) (layer B.Cu) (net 14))
 (segment (start 113.5761 97.3836) (end 113.5761 100.2411) (width 0.5) (layer B.Cu) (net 15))
 (segment (start 113.5761 100.2411) (end 115.57 102.235) (width 0.5) (layer B.Cu) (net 15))
 (segment (start 115.57 102.235) (end 125.095 102.235) (width 0.5) (layer B.Cu) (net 15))
 (segment (start 125.095 102.235) (end 126.365 103.505) (width 0.5) (layer B.Cu) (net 15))
 (segment (start 126.365 103.505) (end 126.365 135.255) (width 0.5) (layer B.Cu) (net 15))
 (segment (start 126.365 135.255) (end 123.825 137.795) (width 0.5) (layer B.Cu) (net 15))
 (segment (start 123.825 137.795) (end 122.1994 137.795) (width 0.5) (layer B.Cu) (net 15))
 (segment (start 122.1994 137.795) (end 121.7422 138.2522) (width 0.5) (layer B.Cu) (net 15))
 (segment (start 116.1161 97.3836) (end 116.1161 100.2411) (width 0.5) (layer B.Cu) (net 16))
 (segment (start 116.1161 100.2411) (end 116.84 100.965) (width 0.5) (layer B.Cu) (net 16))
 (segment (start 116.84 100.965) (end 125.095 100.965) (width 0.5) (layer B.Cu) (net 16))
 (segment (start 125.095 100.965) (end 125.73 100.965) (width 0.5) (layer B.Cu) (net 16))
 (segment (start 125.73 100.965) (end 127 102.235) (width 0.5) (layer B.Cu) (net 16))
 (segment (start 127 102.235) (end 127.635 102.87) (width 0.5) (layer B.Cu) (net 16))
 (segment (start 127.635 102.87) (end 127.635 136.525) (width 0.5) (layer B.Cu) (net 16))
 (segment (start 127.635 136.525) (end 123.3678 140.7922) (width 0.5) (layer B.Cu) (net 16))
 (segment (start 123.3678 140.7922) (end 121.7422 140.7922) (width 0.5) (layer B.Cu) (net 16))
 (segment (start 116.1161 68.8086) (end 116.1161 76.001101) (width 1.6) (layer B.Cu) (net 2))
 (segment (start 116.1161 76.001101) (end 116.205 76.090001) (width 1.6) (layer B.Cu) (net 2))
 (segment (start 121.1961 68.8086) (end 121.1961 76.001101) (width 1.6) (layer B.Cu) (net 4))
 (segment (start 121.1961 76.001101) (end 121.285 76.090001) (width 1.6) (layer B.Cu) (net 4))
 (segment (start 123.825 113.665) (end 118.745 113.665) (width 0.5) (layer B.Cu) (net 6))
 (via (at 118.745 113.665) (size 2) (drill 0.8) (layers F.Cu B.Cu) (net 6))
 (segment (start 118.745 113.665) (end 109.855 113.665) (width 0.5) (layer F.Cu) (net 6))
 (segment (start 108.4961 98.9711) (end 114.3 104.775) (width 0.5) (layer B.Cu) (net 6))
 (segment (start 114.3 104.775) (end 122.555 104.775) (width 0.5) (layer B.Cu) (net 6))
 (segment (start 122.555 104.775) (end 123.825 106.045) (width 0.5) (layer B.Cu) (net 6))
 (segment (start 123.825 106.045) (end 123.825 113.665) (width 0.5) (layer B.Cu) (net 6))
 (segment (start 123.825 113.665) (end 123.825 126.0094) (width 0.5) (layer B.Cu) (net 6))
 (via (at 109.855 113.665) (size 2) (drill 0.8) (layers F.Cu B.Cu) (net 6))
 (segment (start 109.855 113.665) (end 109.855 128.27) (width 0.5) (layer B.Cu) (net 6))
 (segment (start 109.855 128.27) (end 110.49 128.905) (width 0.5) (layer B.Cu) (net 6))
 (segment (start 110.49 128.905) (end 110.49 130.81) (width 0.5) (layer B.Cu) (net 6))
 (segment (start 110.49 130.81) (end 114.935 135.255) (width 0.5) (layer B.Cu) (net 6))
 (segment (start 114.935 135.255) (end 114.935 148.59) (width 0.5) (layer B.Cu) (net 6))
 (segment (start 114.935 148.59) (end 114.815 148.47) (width 0.5) (layer B.Cu) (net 6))
 (segment (start 114.815 148.47) (end 111.125 148.47) (width 0.5) (layer B.Cu) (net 6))
 (segment (start 108.4961 97.3836) (end 108.4961 98.9711) (width 0.5) (layer B.Cu) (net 6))
 (segment (start 123.825 126.0094) (end 121.7422 128.0922) (width 0.5) (layer B.Cu) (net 6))
 (segment (start 108.4961 97.3836) (end 108.4961 90.0811) (width 1.6) (layer B.Cu) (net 6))
 (segment (start 108.4961 90.0811) (end 101.8286 83.4136) (width 1.6) (layer B.Cu) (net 6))
 (segment (start 101.8286 83.4136) (end 100.2411 83.4136) (width 1.6) (layer B.Cu) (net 6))
 (segment (start 111.125 143.47) (end 106.64 143.47) (width 0.5) (layer B.Cu) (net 32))
 (segment (start 106.64 143.47) (end 106.5022 143.3322) (width 0.5) (layer B.Cu) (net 32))
 (segment (start 111.125 145.97) (end 106.6 145.97) (width 0.5) (layer B.Cu) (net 34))
 (segment (start 106.6 145.97) (end 106.5022 145.8722) (width 0.5) (layer B.Cu) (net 34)))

